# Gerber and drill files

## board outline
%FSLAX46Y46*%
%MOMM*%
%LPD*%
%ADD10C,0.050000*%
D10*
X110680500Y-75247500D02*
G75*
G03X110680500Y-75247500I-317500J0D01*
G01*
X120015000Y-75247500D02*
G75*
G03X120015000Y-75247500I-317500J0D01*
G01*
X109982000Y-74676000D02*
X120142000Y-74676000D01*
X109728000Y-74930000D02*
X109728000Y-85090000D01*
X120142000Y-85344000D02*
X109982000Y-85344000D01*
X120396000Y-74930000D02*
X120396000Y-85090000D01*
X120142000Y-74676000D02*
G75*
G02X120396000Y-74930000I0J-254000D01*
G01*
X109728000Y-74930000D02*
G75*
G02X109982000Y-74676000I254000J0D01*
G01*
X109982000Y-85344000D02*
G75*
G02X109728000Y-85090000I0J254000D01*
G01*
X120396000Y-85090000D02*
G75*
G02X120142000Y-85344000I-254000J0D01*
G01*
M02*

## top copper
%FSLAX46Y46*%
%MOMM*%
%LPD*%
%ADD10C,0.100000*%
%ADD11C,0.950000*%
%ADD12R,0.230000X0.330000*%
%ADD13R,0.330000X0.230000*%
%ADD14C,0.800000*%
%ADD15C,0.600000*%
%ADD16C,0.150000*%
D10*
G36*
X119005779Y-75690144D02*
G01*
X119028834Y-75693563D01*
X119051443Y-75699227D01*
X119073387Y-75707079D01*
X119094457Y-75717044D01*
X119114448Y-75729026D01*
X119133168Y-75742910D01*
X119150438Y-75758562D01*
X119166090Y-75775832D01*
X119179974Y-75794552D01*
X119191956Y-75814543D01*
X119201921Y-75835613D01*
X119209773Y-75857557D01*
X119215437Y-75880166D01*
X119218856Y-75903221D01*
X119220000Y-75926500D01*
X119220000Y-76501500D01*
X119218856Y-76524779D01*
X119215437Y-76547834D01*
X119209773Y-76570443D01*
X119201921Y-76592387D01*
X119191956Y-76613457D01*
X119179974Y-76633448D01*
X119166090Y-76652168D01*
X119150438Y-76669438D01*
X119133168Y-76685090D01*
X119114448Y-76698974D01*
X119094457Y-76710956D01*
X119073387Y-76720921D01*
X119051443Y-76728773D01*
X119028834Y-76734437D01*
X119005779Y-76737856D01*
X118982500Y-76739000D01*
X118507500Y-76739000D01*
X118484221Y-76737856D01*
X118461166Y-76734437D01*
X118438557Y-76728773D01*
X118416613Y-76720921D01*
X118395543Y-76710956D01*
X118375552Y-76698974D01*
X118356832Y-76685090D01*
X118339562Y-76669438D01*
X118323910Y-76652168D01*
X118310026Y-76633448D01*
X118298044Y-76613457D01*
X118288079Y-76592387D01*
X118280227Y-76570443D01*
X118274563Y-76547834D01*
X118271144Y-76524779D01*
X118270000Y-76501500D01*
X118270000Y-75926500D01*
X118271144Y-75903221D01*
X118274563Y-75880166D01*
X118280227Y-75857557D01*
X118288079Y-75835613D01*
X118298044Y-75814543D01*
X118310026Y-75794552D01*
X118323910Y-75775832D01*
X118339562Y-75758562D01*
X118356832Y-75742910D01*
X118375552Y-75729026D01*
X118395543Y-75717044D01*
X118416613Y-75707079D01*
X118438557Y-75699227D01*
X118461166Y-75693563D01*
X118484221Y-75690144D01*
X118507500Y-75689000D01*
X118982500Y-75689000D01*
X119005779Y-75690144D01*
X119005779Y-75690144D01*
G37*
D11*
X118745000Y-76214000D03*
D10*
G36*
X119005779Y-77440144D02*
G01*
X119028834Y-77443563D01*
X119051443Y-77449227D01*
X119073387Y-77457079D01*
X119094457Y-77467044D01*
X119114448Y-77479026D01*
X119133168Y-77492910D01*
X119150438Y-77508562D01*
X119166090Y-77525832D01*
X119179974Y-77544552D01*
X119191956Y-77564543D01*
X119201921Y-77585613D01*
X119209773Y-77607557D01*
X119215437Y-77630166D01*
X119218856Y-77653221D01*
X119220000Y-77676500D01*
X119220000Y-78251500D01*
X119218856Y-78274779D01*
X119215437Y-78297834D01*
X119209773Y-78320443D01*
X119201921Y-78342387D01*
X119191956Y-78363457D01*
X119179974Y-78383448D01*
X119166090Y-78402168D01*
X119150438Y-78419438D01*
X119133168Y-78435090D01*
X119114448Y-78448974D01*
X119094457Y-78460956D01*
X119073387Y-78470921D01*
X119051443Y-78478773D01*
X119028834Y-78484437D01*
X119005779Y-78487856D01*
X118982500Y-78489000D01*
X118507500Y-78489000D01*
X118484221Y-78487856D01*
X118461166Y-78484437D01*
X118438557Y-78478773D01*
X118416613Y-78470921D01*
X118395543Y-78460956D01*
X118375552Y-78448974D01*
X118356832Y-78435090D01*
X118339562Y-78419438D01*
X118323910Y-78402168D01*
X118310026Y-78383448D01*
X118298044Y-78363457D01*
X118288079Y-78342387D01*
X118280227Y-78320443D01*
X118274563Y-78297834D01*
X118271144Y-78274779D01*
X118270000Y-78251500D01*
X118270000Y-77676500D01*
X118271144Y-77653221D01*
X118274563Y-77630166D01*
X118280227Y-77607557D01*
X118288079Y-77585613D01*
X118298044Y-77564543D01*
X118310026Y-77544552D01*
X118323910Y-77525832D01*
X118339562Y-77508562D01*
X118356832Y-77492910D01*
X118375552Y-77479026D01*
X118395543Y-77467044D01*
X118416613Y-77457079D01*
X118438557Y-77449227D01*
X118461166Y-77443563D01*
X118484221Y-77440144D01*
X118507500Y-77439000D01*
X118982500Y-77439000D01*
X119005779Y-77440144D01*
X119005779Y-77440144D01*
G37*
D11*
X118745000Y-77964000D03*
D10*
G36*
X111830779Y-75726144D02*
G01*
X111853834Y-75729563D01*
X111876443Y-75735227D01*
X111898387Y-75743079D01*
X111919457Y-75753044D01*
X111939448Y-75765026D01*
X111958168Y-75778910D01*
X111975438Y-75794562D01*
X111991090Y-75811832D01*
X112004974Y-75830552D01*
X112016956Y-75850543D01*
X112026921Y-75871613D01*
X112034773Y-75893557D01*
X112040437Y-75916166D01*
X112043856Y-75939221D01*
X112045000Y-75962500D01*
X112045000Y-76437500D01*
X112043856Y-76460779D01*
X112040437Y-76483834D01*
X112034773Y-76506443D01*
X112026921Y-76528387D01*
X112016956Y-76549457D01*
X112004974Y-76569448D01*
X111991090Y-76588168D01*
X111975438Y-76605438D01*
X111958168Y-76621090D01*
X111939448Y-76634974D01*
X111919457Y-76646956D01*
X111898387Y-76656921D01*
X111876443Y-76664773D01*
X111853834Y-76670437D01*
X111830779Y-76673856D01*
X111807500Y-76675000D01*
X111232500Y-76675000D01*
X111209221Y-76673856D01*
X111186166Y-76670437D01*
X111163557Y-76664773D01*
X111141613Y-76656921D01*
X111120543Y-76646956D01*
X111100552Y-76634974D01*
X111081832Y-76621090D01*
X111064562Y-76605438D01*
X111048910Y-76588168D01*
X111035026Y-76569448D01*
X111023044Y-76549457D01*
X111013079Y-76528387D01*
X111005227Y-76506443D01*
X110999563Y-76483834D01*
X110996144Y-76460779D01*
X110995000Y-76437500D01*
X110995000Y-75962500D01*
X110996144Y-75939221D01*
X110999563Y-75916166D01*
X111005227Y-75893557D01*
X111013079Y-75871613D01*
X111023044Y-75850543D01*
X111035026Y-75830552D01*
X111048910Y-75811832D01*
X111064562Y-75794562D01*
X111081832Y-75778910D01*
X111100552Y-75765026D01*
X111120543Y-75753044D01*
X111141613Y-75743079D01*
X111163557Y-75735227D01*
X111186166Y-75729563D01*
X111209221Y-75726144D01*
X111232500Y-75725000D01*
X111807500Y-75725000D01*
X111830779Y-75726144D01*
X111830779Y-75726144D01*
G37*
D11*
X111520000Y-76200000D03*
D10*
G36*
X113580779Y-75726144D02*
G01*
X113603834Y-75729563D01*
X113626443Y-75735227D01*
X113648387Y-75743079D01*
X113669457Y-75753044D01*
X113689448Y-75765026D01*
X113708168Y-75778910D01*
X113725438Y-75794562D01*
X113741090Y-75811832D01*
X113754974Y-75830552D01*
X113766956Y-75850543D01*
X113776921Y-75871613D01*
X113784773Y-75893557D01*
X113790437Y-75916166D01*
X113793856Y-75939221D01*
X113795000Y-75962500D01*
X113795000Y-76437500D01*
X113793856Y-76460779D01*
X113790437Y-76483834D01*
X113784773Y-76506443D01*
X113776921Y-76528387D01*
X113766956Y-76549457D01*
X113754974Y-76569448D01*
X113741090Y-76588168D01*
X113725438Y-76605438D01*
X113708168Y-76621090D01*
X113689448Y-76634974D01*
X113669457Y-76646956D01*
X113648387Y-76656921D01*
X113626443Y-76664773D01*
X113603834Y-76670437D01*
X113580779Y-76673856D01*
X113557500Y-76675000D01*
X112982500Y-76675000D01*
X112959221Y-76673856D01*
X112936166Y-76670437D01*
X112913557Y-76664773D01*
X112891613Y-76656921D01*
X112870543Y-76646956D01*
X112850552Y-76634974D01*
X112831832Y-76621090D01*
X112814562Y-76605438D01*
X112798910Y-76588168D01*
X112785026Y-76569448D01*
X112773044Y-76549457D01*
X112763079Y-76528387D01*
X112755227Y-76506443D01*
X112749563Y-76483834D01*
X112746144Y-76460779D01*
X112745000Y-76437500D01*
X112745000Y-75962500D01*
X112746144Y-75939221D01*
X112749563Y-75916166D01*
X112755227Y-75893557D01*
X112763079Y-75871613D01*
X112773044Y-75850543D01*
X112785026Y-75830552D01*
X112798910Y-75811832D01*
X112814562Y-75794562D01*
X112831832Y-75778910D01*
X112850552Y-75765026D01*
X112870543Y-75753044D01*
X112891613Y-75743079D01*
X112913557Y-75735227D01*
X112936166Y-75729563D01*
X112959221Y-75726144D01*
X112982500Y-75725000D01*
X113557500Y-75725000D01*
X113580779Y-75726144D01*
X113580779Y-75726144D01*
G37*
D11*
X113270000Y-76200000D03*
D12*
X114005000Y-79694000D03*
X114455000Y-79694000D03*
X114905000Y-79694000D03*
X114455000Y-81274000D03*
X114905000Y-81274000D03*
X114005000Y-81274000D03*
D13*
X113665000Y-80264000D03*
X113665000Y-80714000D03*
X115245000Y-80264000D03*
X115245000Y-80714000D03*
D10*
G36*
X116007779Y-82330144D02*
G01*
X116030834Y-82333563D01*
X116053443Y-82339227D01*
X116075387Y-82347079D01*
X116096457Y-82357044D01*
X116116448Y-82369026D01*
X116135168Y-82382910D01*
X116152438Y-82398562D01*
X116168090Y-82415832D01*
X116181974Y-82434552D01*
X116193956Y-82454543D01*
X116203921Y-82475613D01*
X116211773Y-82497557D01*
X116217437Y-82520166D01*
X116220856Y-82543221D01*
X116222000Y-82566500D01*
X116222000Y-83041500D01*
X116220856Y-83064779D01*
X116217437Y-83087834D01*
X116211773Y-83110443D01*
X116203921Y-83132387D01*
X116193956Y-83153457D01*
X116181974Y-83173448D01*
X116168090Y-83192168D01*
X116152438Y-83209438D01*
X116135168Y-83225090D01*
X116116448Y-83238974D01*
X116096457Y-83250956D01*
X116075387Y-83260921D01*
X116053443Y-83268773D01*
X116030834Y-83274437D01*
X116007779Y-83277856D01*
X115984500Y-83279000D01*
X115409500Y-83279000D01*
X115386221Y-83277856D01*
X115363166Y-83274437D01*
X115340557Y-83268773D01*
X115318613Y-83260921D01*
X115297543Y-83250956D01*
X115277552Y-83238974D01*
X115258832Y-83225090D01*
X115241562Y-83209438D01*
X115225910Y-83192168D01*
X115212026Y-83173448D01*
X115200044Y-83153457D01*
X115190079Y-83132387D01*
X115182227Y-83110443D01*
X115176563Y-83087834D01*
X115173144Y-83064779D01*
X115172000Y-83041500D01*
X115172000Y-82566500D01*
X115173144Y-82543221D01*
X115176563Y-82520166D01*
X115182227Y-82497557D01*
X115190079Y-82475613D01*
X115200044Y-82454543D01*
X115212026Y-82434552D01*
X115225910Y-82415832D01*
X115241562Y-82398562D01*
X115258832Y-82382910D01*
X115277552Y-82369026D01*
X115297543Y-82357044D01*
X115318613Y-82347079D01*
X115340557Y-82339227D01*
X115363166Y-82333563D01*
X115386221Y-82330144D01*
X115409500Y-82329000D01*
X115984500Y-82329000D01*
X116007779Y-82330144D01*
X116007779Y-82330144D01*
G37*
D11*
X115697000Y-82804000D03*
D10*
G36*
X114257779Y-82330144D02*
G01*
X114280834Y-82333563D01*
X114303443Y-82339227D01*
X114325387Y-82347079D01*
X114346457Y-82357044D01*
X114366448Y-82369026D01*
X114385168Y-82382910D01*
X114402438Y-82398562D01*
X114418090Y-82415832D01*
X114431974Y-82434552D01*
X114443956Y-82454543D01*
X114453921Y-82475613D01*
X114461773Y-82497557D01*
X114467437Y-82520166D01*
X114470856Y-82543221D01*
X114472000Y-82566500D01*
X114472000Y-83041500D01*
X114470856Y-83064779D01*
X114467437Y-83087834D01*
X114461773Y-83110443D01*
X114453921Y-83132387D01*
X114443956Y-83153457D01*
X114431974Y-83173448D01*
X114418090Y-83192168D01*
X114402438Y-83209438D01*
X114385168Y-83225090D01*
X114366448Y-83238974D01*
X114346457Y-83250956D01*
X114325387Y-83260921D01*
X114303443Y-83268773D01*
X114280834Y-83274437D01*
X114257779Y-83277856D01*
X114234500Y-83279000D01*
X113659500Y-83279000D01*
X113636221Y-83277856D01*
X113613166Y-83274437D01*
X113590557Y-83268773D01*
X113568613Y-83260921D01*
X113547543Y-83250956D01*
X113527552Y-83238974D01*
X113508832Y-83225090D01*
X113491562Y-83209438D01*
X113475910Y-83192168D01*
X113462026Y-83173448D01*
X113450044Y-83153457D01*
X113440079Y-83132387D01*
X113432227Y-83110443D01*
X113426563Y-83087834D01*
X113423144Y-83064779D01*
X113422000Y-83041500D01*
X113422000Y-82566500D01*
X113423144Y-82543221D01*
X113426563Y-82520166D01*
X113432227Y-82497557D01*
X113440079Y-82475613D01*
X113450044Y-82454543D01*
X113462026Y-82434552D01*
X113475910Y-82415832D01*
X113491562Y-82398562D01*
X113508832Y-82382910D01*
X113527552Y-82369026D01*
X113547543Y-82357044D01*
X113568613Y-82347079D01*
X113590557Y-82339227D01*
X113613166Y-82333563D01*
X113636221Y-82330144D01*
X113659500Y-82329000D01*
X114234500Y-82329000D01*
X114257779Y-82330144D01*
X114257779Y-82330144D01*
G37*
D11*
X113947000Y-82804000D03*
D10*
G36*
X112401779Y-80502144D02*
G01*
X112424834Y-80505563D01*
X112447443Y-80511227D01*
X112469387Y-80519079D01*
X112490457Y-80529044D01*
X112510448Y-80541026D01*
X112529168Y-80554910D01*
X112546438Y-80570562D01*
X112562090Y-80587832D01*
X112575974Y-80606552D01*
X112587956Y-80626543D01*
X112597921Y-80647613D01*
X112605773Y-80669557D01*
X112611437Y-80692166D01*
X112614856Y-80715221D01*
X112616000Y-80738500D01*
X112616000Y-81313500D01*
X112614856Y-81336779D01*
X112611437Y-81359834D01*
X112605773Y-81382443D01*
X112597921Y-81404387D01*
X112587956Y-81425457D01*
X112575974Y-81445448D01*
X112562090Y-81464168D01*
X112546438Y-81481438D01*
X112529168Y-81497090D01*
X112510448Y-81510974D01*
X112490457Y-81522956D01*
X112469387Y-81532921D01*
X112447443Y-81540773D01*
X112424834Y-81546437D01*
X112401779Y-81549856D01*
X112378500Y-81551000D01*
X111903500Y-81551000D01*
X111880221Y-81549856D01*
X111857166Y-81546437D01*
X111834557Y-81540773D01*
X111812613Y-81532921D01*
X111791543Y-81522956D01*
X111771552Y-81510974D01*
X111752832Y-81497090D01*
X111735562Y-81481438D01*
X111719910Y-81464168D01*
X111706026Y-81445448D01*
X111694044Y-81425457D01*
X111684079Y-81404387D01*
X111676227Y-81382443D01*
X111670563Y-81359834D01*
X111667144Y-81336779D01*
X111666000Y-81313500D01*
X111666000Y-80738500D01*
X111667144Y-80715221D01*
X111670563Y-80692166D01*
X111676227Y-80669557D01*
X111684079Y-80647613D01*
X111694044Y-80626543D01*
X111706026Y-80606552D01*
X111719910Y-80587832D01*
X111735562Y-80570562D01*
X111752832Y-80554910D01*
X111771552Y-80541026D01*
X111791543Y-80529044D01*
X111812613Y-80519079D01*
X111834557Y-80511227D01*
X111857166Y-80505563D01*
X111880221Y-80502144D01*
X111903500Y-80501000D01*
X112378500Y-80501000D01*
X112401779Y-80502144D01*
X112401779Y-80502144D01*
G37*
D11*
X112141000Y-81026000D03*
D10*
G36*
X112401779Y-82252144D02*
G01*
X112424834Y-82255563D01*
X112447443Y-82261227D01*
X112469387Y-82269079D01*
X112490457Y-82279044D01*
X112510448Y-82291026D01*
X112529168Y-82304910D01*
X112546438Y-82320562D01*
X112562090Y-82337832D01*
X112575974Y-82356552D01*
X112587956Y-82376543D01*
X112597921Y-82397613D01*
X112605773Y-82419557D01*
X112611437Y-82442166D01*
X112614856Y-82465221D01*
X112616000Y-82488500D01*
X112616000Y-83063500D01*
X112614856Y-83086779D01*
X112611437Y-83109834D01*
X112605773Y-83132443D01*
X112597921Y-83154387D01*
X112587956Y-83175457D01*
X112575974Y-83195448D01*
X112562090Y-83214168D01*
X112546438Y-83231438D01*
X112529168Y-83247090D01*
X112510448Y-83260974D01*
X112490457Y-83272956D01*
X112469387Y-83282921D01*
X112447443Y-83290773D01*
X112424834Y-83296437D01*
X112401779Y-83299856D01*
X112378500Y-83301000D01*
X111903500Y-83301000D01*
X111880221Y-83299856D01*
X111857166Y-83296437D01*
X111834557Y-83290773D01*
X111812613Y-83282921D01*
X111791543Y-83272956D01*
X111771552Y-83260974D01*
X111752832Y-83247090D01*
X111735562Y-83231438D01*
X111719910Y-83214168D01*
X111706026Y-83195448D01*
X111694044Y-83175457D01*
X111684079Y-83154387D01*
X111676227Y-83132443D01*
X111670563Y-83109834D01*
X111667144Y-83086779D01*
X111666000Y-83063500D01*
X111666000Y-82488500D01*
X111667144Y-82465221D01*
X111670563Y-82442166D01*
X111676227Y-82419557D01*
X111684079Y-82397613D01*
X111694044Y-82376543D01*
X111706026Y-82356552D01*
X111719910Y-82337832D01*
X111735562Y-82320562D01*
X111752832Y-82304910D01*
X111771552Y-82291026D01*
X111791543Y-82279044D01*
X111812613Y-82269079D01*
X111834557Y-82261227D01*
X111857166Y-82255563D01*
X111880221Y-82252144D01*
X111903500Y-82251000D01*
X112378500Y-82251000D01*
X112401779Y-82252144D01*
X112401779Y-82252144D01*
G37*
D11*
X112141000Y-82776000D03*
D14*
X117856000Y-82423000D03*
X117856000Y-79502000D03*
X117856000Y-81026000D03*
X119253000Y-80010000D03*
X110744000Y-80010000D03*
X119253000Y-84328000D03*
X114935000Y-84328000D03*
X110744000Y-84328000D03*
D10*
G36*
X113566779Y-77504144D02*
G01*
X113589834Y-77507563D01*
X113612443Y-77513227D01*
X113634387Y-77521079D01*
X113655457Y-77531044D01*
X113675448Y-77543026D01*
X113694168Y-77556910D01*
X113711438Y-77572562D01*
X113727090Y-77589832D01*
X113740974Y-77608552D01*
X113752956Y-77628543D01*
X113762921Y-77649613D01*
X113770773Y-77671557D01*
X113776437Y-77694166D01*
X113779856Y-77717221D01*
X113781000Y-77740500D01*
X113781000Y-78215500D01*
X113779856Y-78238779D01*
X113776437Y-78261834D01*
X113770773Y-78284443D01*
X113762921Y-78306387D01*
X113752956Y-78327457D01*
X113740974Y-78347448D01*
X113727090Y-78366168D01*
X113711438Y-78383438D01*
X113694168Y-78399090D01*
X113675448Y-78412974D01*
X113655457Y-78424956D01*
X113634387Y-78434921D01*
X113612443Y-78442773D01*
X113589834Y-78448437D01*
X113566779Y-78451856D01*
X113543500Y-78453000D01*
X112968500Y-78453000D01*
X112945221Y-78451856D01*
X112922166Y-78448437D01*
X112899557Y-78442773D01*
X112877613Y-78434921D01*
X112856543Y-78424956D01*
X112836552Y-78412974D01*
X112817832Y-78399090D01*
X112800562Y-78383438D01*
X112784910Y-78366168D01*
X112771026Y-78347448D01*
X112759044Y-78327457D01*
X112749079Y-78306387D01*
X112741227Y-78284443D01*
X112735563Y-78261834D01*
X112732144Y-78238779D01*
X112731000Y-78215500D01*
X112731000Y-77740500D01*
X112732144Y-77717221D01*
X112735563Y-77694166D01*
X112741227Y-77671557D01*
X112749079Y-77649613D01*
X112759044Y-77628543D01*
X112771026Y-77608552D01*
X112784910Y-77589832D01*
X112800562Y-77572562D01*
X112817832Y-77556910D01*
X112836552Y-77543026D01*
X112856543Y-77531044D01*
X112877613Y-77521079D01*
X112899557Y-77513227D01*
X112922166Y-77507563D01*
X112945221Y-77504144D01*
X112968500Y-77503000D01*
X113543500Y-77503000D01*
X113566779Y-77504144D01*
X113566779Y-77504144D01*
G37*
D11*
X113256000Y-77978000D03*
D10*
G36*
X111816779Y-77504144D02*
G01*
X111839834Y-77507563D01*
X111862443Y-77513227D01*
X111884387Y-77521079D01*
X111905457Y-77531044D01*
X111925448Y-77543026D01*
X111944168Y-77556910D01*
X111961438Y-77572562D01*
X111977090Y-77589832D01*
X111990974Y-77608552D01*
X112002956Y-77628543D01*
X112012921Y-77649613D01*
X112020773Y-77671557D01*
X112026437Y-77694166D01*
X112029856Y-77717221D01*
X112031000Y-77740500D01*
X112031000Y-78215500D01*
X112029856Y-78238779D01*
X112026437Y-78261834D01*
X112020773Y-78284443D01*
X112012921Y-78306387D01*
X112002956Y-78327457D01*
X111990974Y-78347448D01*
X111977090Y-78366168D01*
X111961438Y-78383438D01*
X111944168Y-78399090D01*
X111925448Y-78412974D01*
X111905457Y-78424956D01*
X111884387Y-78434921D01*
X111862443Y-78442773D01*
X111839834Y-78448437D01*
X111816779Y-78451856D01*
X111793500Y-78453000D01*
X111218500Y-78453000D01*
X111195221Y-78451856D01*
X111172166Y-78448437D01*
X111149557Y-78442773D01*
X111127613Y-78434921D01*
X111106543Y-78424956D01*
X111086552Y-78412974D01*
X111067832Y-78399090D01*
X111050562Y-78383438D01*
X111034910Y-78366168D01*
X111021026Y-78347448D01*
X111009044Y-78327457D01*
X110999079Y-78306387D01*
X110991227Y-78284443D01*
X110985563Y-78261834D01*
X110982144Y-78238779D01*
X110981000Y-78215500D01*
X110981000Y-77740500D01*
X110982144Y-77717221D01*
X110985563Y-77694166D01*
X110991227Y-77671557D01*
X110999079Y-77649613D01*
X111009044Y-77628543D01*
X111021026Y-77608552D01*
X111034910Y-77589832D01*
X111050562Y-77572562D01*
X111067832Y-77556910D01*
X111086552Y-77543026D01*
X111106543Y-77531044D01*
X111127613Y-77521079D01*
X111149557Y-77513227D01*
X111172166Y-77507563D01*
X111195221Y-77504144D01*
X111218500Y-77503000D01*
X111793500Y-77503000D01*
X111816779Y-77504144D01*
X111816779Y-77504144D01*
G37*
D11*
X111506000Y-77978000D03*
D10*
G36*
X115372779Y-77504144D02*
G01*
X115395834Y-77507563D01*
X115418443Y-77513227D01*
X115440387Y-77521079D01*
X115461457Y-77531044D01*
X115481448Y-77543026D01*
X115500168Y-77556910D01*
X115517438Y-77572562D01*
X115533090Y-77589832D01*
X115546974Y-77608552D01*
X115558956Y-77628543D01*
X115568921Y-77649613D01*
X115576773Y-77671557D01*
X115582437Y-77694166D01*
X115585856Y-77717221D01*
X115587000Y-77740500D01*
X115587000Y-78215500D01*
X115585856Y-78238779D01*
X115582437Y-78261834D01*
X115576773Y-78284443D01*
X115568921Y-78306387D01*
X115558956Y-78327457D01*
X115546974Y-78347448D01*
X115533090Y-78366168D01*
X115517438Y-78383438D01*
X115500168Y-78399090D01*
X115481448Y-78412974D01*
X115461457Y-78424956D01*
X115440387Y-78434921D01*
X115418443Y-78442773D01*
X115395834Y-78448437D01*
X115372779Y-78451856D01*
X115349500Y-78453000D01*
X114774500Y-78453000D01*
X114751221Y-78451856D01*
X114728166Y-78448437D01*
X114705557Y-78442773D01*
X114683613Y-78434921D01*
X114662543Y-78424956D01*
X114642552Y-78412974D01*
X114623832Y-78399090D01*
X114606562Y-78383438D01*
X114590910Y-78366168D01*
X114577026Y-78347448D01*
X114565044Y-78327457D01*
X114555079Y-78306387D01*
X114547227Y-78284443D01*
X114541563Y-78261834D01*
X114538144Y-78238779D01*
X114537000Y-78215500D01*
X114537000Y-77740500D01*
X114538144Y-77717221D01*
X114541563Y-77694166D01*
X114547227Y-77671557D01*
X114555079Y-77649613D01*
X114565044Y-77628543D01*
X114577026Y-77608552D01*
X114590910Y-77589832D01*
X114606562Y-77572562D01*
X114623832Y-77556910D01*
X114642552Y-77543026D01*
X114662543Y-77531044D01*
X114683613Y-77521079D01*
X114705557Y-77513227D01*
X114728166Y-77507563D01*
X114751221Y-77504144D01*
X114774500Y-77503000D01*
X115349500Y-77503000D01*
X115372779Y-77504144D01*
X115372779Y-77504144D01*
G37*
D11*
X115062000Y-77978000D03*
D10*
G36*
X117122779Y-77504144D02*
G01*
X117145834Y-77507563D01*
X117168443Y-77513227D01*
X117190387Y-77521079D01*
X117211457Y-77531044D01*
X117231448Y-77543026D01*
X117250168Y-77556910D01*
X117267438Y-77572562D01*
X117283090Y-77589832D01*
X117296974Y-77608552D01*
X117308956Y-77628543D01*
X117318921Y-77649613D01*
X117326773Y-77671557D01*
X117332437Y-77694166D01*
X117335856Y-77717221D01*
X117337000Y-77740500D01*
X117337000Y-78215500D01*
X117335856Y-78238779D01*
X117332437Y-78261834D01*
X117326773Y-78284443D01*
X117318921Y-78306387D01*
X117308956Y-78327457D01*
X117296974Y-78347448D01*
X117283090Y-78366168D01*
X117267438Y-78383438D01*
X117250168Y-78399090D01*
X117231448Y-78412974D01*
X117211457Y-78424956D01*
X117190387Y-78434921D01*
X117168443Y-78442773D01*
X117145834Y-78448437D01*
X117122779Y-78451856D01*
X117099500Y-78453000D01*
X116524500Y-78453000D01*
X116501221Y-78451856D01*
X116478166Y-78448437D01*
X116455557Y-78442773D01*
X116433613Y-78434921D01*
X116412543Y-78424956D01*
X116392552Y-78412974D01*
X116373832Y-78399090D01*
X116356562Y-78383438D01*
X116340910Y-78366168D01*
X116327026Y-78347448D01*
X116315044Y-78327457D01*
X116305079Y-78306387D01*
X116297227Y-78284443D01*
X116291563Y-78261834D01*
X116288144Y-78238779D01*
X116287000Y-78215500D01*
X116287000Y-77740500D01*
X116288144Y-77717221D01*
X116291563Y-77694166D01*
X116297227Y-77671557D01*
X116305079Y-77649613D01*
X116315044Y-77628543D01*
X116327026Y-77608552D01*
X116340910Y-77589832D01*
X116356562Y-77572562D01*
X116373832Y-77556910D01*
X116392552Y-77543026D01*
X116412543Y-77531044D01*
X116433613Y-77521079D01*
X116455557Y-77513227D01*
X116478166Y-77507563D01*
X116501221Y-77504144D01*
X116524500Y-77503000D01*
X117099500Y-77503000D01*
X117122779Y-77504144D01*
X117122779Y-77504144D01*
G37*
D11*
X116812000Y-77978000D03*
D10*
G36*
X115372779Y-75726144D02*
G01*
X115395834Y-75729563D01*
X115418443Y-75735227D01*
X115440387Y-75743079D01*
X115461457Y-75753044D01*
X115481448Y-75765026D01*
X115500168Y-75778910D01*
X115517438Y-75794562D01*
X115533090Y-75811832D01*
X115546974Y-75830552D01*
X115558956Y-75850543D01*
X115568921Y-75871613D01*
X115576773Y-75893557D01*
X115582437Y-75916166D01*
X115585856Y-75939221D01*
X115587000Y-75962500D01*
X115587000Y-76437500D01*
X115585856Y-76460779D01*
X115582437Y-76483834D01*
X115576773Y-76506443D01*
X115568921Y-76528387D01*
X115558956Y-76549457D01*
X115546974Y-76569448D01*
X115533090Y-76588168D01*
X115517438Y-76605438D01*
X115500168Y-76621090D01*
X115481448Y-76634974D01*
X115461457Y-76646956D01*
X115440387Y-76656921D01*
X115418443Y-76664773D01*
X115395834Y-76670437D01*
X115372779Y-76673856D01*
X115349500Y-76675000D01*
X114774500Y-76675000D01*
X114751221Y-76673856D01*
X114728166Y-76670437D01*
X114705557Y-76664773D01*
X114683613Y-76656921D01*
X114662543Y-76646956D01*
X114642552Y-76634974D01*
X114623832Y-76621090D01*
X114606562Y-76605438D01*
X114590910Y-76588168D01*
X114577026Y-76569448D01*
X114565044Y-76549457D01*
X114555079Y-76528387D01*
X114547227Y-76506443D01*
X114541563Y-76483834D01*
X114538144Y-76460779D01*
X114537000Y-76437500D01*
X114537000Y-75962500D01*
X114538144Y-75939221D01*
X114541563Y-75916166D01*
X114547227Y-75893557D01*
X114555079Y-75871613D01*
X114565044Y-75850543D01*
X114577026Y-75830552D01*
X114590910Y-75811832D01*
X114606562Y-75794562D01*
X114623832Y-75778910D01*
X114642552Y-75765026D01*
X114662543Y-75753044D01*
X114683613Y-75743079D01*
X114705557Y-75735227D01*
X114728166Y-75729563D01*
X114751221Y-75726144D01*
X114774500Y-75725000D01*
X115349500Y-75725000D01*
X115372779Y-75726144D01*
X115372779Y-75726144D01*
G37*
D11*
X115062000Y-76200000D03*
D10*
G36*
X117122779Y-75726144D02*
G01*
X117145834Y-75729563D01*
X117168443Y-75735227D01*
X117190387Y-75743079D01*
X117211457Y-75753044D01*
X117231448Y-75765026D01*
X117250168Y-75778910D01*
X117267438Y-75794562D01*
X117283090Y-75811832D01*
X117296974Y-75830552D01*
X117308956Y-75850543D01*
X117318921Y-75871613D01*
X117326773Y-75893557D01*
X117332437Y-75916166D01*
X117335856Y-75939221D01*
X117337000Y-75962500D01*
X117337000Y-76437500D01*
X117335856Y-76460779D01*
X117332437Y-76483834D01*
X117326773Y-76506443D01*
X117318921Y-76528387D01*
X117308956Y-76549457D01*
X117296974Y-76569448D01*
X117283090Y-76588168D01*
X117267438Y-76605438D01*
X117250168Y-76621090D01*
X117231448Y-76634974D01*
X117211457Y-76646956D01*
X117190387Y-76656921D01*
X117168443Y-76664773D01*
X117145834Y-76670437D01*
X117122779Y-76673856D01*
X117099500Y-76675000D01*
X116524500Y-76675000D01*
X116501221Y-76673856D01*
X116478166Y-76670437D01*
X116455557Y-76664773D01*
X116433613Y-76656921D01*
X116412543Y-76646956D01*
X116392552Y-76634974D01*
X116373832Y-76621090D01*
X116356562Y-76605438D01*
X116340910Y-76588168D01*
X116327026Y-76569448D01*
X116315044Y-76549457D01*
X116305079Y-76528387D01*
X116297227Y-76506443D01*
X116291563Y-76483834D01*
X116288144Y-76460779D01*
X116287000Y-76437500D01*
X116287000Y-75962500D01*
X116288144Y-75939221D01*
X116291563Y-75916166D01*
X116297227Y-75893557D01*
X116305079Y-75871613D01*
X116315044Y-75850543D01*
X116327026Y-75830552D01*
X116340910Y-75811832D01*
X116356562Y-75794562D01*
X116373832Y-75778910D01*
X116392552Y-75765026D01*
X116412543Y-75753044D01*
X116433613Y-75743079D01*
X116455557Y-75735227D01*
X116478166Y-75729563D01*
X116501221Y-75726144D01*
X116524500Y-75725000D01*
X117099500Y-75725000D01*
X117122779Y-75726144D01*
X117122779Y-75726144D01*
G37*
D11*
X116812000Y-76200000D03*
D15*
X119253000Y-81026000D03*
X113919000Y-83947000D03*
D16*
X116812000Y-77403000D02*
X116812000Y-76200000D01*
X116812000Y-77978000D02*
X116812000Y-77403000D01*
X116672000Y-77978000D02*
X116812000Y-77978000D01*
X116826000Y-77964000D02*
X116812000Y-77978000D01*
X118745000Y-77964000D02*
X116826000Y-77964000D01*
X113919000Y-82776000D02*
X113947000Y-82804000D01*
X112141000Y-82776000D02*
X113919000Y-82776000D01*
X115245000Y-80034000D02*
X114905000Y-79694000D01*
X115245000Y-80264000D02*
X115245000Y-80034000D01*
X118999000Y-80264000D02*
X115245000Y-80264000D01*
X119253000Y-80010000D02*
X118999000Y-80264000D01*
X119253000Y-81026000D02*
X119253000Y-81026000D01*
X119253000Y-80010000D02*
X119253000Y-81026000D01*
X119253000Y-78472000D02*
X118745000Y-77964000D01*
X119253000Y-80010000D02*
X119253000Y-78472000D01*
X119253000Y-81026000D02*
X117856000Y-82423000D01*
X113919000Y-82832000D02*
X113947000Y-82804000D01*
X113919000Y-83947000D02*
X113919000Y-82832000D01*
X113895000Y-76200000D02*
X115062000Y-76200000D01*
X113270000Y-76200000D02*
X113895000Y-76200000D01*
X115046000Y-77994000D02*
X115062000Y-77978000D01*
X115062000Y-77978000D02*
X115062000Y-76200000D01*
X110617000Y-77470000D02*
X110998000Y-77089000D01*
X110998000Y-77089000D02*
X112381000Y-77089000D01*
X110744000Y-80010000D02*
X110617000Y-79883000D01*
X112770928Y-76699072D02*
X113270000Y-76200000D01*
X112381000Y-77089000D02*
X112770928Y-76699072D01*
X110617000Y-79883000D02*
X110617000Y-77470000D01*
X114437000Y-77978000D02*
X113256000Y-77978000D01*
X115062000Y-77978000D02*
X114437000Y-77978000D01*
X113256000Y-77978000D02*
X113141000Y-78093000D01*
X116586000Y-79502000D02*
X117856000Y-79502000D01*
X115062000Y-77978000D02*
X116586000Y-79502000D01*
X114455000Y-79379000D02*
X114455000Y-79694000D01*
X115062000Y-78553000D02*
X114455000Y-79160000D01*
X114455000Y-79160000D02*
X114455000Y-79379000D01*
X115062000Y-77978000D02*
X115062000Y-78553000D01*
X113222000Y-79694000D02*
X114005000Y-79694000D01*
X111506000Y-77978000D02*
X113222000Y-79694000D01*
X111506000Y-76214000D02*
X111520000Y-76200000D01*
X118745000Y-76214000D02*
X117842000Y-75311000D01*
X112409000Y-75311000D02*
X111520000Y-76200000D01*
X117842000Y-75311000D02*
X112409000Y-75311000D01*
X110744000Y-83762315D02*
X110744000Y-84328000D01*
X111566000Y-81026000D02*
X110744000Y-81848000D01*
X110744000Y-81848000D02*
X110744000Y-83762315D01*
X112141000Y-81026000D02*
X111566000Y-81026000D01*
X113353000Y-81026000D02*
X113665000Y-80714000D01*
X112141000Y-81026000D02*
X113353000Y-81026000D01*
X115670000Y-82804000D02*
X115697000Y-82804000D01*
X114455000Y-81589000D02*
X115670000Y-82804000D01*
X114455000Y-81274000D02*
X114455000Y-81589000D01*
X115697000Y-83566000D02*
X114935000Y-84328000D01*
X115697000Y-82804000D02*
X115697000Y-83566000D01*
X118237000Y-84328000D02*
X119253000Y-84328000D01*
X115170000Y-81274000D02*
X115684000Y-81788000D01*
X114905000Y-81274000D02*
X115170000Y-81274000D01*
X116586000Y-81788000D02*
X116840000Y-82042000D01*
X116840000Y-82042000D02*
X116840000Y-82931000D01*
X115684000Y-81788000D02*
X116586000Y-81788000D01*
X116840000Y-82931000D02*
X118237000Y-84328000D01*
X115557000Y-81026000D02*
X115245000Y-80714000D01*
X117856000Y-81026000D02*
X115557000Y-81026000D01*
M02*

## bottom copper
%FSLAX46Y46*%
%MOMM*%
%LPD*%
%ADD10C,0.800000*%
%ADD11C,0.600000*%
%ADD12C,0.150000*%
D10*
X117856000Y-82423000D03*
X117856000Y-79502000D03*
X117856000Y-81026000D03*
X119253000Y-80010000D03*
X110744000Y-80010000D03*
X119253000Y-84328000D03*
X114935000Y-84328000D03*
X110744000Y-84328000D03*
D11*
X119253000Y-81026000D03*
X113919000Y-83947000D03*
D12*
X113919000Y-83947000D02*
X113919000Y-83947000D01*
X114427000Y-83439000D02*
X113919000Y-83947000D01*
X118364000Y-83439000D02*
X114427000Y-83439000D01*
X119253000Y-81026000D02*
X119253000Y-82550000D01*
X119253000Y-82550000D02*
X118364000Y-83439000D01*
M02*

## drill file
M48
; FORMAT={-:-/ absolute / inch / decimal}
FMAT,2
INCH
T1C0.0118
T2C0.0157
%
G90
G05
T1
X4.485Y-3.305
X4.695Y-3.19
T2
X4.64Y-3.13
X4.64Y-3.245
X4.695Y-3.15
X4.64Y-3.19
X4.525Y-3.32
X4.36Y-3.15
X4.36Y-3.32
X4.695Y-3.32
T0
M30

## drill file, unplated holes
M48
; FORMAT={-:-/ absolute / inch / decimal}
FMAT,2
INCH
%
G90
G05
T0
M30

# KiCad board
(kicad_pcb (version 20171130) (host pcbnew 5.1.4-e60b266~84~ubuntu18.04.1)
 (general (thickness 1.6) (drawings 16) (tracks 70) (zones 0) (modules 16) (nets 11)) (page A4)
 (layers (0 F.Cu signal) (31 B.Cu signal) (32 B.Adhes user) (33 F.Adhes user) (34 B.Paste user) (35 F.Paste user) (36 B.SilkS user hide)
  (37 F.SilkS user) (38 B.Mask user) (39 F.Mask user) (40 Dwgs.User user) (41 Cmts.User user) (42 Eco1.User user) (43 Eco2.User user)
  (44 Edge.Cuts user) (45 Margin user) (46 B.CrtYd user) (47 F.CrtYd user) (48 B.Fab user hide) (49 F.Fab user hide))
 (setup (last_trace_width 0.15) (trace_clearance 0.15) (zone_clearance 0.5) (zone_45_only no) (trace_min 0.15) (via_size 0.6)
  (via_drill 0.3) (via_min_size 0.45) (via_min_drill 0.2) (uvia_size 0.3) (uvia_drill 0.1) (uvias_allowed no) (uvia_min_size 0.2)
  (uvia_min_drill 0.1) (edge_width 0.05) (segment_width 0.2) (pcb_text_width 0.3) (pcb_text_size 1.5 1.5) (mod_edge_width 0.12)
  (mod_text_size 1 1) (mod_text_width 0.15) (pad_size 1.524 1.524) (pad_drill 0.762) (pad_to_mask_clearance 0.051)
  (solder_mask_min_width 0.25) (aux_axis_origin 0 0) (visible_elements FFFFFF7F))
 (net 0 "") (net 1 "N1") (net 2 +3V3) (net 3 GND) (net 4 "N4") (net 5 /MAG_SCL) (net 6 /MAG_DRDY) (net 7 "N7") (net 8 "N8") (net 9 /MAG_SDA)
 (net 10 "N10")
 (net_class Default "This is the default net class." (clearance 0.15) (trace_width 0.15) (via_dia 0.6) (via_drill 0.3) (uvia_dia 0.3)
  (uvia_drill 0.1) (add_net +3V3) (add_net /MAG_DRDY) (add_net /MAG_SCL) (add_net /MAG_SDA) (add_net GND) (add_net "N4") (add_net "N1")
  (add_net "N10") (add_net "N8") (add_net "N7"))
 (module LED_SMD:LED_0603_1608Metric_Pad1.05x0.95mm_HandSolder (layer F.Cu) (at 118.745 77.089 270)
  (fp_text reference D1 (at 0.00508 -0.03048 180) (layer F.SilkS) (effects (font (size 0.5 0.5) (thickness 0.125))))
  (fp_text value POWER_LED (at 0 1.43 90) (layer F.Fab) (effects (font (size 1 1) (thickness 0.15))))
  (pad 1 smd roundrect (at -0.875 0 270) (size 1.05 0.95) (layers F.Cu F.Paste F.Mask) (roundrect_rratio 0.25) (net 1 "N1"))
  (pad 2 smd roundrect (at 0.875 0 270) (size 1.05 0.95) (layers F.Cu F.Paste F.Mask) (roundrect_rratio 0.25) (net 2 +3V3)))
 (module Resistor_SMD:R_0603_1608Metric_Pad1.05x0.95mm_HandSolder (layer F.Cu) (at 112.395 76.2)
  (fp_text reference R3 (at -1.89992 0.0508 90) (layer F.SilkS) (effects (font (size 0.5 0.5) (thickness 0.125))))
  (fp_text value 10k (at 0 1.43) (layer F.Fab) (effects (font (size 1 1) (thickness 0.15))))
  (pad 1 smd roundrect (at -0.875 0) (size 1.05 0.95) (layers F.Cu F.Paste F.Mask) (roundrect_rratio 0.25) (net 1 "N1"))
  (pad 2 smd roundrect (at 0.875 0) (size 1.05 0.95) (layers F.Cu F.Paste F.Mask) (roundrect_rratio 0.25) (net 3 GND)))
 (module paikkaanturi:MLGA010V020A (layer F.Cu) (at 113.455 79.484)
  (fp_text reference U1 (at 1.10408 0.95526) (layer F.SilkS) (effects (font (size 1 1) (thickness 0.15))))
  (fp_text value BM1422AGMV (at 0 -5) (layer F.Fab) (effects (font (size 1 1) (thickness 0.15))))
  (pad 3 smd rect (at 0.55 0.21) (size 0.23 0.33) (layers F.Cu F.Paste F.Mask) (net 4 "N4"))
  (pad 2 smd rect (at 1 0.21) (size 0.23 0.33) (layers F.Cu F.Paste F.Mask) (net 3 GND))
  (pad 1 smd rect (at 1.45 0.21) (size 0.23 0.33) (layers F.Cu F.Paste F.Mask) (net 2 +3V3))
  (pad 7 smd rect (at 1 1.79) (size 0.23 0.33) (layers F.Cu F.Paste F.Mask) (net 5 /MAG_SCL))
  (pad 8 smd rect (at 1.45 1.79) (size 0.23 0.33) (layers F.Cu F.Paste F.Mask) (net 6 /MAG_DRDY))
  (pad 6 smd rect (at 0.55 1.79) (size 0.23 0.33) (layers F.Cu F.Paste F.Mask) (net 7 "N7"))
  (pad 4 smd rect (at 0.21 0.78 90) (size 0.23 0.33) (layers F.Cu F.Paste F.Mask) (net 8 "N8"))
  (pad 5 smd rect (at 0.21 1.23 90) (size 0.23 0.33) (layers F.Cu F.Paste F.Mask) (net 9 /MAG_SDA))
  (pad 10 smd rect (at 1.79 0.78 90) (size 0.23 0.33) (layers F.Cu F.Paste F.Mask) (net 2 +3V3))
  (pad 9 smd rect (at 1.79 1.23 90) (size 0.23 0.33) (layers F.Cu F.Paste F.Mask) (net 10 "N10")))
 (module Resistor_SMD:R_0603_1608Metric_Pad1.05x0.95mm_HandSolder (layer F.Cu) (at 114.822 82.804 180)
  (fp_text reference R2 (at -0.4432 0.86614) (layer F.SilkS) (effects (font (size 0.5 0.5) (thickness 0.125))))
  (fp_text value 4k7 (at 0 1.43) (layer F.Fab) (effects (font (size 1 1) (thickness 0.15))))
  (pad 1 smd roundrect (at -0.875 0 180) (size 1.05 0.95) (layers F.Cu F.Paste F.Mask) (roundrect_rratio 0.25) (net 5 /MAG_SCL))
  (pad 2 smd roundrect (at 0.875 0 180) (size 1.05 0.95) (layers F.Cu F.Paste F.Mask) (roundrect_rratio 0.25) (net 2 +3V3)))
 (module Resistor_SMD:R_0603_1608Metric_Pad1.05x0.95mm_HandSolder (layer F.Cu) (at 112.141 81.901 270)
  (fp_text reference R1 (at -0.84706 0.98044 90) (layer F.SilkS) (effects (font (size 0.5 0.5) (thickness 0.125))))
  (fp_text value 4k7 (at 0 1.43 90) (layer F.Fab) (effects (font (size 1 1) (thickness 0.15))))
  (pad 1 smd roundrect (at -0.875 0 270) (size 1.05 0.95) (layers F.Cu F.Paste F.Mask) (roundrect_rratio 0.25) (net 9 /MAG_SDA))
  (pad 2 smd roundrect (at 0.875 0 270) (size 1.05 0.95) (layers F.Cu F.Paste F.Mask) (roundrect_rratio 0.25) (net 2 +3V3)))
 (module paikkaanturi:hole (layer F.Cu) (at 117.856 82.423)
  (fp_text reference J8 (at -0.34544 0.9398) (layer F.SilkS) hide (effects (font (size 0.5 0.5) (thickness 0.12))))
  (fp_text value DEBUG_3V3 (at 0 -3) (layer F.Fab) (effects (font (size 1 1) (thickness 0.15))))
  (pad 1 thru_hole circle (at 0 0) (size 0.8 0.8) (drill 0.4) (layers *.Cu *.Mask) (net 2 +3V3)))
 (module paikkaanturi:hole (layer F.Cu) (at 117.856 79.502)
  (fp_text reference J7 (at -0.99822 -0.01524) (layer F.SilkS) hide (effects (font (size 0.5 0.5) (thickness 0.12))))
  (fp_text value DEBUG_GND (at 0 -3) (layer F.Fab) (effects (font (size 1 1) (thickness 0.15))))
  (pad 1 thru_hole circle (at 0 0) (size 0.8 0.8) (drill 0.4) (layers *.Cu *.Mask) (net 3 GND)))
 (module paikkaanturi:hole (layer F.Cu) (at 117.856 81.026)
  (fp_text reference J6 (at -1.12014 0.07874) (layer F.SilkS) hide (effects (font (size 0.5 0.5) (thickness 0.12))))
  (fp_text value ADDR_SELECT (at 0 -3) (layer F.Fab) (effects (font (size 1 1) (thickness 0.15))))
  (pad 1 thru_hole circle (at 0 0) (size 0.8 0.8) (drill 0.4) (layers *.Cu *.Mask) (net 10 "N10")))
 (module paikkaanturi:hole (layer F.Cu) (at 119.253 80.01)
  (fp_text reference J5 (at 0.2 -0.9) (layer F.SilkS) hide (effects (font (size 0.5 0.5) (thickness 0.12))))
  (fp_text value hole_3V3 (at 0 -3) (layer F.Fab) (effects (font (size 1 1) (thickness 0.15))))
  (pad 1 thru_hole circle (at 0 0) (size 0.8 0.8) (drill 0.4) (layers *.Cu *.Mask) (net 2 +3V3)))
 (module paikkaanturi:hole (layer F.Cu) (at 110.744 80.01)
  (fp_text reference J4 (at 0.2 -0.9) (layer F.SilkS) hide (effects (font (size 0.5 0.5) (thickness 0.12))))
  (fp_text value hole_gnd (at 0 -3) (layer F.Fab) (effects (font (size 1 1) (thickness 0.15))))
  (pad 1 thru_hole circle (at 0 0) (size 0.8 0.8) (drill 0.4) (layers *.Cu *.Mask) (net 3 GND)))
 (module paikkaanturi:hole (layer F.Cu) (at 119.253 84.328)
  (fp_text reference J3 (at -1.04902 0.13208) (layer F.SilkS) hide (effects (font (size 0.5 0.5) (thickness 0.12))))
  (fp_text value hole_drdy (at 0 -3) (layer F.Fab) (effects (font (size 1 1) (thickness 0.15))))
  (pad 1 thru_hole circle (at 0 0) (size 0.8 0.8) (drill 0.4) (layers *.Cu *.Mask) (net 6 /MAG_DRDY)))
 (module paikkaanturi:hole (layer F.Cu) (at 114.935 84.328)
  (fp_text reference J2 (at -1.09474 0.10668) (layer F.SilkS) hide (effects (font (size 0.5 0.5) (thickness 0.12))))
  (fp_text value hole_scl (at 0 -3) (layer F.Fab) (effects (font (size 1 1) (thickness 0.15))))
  (pad 1 thru_hole circle (at 0 0) (size 0.8 0.8) (drill 0.4) (layers *.Cu *.Mask) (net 5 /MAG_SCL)))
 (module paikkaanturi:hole (layer F.Cu) (at 110.744 84.328)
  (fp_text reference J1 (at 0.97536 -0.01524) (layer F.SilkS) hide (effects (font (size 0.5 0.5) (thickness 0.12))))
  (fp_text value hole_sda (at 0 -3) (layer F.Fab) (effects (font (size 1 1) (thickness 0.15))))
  (pad 1 thru_hole circle (at 0 0) (size 0.8 0.8) (drill 0.4) (layers *.Cu *.Mask) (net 9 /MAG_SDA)))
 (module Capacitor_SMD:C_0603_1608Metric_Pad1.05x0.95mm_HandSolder (layer F.Cu) (at 112.381 77.978 180)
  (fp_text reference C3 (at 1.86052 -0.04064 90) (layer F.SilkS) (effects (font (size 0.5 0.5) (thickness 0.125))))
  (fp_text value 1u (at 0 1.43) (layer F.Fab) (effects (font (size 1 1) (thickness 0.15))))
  (pad 1 smd roundrect (at -0.875 0 180) (size 1.05 0.95) (layers F.Cu F.Paste F.Mask) (roundrect_rratio 0.25) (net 3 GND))
  (pad 2 smd roundrect (at 0.875 0 180) (size 1.05 0.95) (layers F.Cu F.Paste F.Mask) (roundrect_rratio 0.25) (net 4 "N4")))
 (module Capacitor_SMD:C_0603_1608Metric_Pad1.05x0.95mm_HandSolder (layer F.Cu) (at 115.937 77.978)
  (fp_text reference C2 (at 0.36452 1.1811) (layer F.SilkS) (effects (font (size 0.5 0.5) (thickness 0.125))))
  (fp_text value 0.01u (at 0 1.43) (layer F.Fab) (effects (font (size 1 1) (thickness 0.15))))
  (pad 1 smd roundrect (at -0.875 0) (size 1.05 0.95) (layers F.Cu F.Paste F.Mask) (roundrect_rratio 0.25) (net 3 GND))
  (pad 2 smd roundrect (at 0.875 0) (size 1.05 0.95) (layers F.Cu F.Paste F.Mask) (roundrect_rratio 0.25) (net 2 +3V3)))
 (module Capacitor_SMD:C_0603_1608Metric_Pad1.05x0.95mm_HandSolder (layer F.Cu) (at 115.937 76.2)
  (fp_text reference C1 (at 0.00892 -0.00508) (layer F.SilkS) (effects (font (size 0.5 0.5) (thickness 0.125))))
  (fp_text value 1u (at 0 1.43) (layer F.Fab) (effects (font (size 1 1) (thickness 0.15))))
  (pad 1 smd roundrect (at -0.875 0) (size 1.05 0.95) (layers F.Cu F.Paste F.Mask) (roundrect_rratio 0.25) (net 3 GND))
  (pad 2 smd roundrect (at 0.875 0) (size 1.05 0.95) (layers F.Cu F.Paste F.Mask) (roundrect_rratio 0.25) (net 2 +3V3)))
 (gr_circle (center 110.363 75.2475) (end 110.617 75.057) (layer Edge.Cuts) (width 0.05))
 (gr_circle (center 119.6975 75.2475) (end 119.9515 75.057) (layer Edge.Cuts) (width 0.05))
 (gr_line (start 109.982 74.676) (end 120.142 74.676) (layer Edge.Cuts) (width 0.05))
 (gr_line (start 109.728 74.93) (end 109.728 85.09) (layer Edge.Cuts) (width 0.05))
 (gr_line (start 120.142 85.344) (end 109.982 85.344) (layer Edge.Cuts) (width 0.05))
 (gr_line (start 120.396 74.93) (end 120.396 85.09) (layer Edge.Cuts) (width 0.05))
 (gr_arc (start 120.142 74.93) (end 120.396 74.93) (angle -90) (layer Edge.Cuts) (width 0.05))
 (gr_arc (start 109.982 74.93) (end 109.982 74.676) (angle -90) (layer Edge.Cuts) (width 0.05))
 (gr_arc (start 109.982 85.09) (end 109.728 85.09) (angle -90) (layer Edge.Cuts) (width 0.05))
 (gr_arc (start 120.142 85.09) (end 120.142 85.344) (angle -90) (layer Edge.Cuts) (width 0.05))
 (segment (start 116.812 77.403) (end 116.812 76.2) (width 0.15) (layer F.Cu) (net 2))
 (segment (start 116.812 77.978) (end 116.812 77.403) (width 0.15) (layer F.Cu) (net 2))
 (segment (start 116.672 77.978) (end 116.812 77.978) (width 0.15) (layer F.Cu) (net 2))
 (segment (start 116.826 77.964) (end 116.812 77.978) (width 0.15) (layer F.Cu) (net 2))
 (segment (start 118.745 77.964) (end 116.826 77.964) (width 0.15) (layer F.Cu) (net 2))
 (segment (start 113.919 82.776) (end 113.947 82.804) (width 0.15) (layer F.Cu) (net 2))
 (segment (start 112.141 82.776) (end 113.919 82.776) (width 0.15) (layer F.Cu) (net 2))
 (segment (start 115.245 80.034) (end 114.905 79.694) (width 0.15) (layer F.Cu) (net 2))
 (segment (start 115.245 80.264) (end 115.245 80.034) (width 0.15) (layer F.Cu) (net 2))
 (segment (start 118.999 80.264) (end 115.245 80.264) (width 0.15) (layer F.Cu) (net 2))
 (segment (start 119.253 80.01) (end 118.999 80.264) (width 0.15) (layer F.Cu) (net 2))
 (segment (start 119.253 81.026) (end 119.253 81.026) (width 0.15) (layer F.Cu) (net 2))
 (segment (start 119.253 80.01) (end 119.253 81.026) (width 0.15) (layer F.Cu) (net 2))
 (segment (start 119.253 78.472) (end 118.745 77.964) (width 0.15) (layer F.Cu) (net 2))
 (segment (start 119.253 80.01) (end 119.253 78.472) (width 0.15) (layer F.Cu) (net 2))
 (segment (start 119.253 81.026) (end 117.856 82.423) (width 0.15) (layer F.Cu) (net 2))
 (via (at 119.253 81.026) (size 0.6) (drill 0.3) (layers F.Cu B.Cu) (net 2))
 (segment (start 113.919 83.947) (end 113.919 83.947) (width 0.15) (layer B.Cu) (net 2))
 (via (at 113.919 83.947) (size 0.6) (drill 0.3) (layers F.Cu B.Cu) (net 2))
 (segment (start 113.919 82.832) (end 113.947 82.804) (width 0.15) (layer F.Cu) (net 2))
 (segment (start 113.919 83.947) (end 113.919 82.832) (width 0.15) (layer F.Cu) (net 2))
 (segment (start 114.427 83.439) (end 113.919 83.947) (width 0.15) (layer B.Cu) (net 2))
 (segment (start 118.364 83.439) (end 114.427 83.439) (width 0.15) (layer B.Cu) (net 2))
 (segment (start 119.253 81.026) (end 119.253 82.55) (width 0.15) (layer B.Cu) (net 2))
 (segment (start 119.253 82.55) (end 118.364 83.439) (width 0.15) (layer B.Cu) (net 2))
 (segment (start 113.895 76.2) (end 115.062 76.2) (width 0.15) (layer F.Cu) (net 3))
 (segment (start 113.27 76.2) (end 113.895 76.2) (width 0.15) (layer F.Cu) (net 3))
 (segment (start 115.046 77.994) (end 115.062 77.978) (width 0.15) (layer F.Cu) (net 3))
 (segment (start 115.062 77.978) (end 115.062 76.2) (width 0.15) (layer F.Cu) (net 3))
 (segment (start 110.617 77.47) (end 110.998 77.089) (width 0.15) (layer F.Cu) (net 3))
 (segment (start 110.998 77.089) (end 112.381 77.089) (width 0.15) (layer F.Cu) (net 3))
 (segment (start 110.744 80.01) (end 110.617 79.883) (width 0.15) (layer F.Cu) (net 3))
 (segment (start 112.770928 76.699072) (end 113.27 76.2) (width 0.15) (layer F.Cu) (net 3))
 (segment (start 112.381 77.089) (end 112.770928 76.699072) (width 0.15) (layer F.Cu) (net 3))
 (segment (start 110.617 79.883) (end 110.617 77.47) (width 0.15) (layer F.Cu) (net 3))
 (segment (start 114.437 77.978) (end 113.256 77.978) (width 0.15) (layer F.Cu) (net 3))
 (segment (start 115.062 77.978) (end 114.437 77.978) (width 0.15) (layer F.Cu) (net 3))
 (segment (start 113.256 77.978) (end 113.141 78.093) (width 0.15) (layer F.Cu) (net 3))
 (segment (start 116.586 79.502) (end 117.856 79.502) (width 0.15) (layer F.Cu) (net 3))
 (segment (start 115.062 77.978) (end 116.586 79.502) (width 0.15) (layer F.Cu) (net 3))
 (segment (start 114.455 79.379) (end 114.455 79.694) (width 0.15) (layer F.Cu) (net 3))
 (segment (start 115.062 78.553) (end 114.455 79.16) (width 0.15) (layer F.Cu) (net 3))
 (segment (start 114.455 79.16) (end 114.455 79.379) (width 0.15) (layer F.Cu) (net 3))
 (segment (start 115.062 77.978) (end 115.062 78.553) (width 0.15) (layer F.Cu) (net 3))
 (segment (start 113.222 79.694) (end 114.005 79.694) (width 0.15) (layer F.Cu) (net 4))
 (segment (start 111.506 77.978) (end 113.222 79.694) (width 0.15) (layer F.Cu) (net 4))
 (segment (start 111.506 76.214) (end 111.52 76.2) (width 0.15) (layer F.Cu) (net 1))
 (segment (start 118.745 76.214) (end 117.842 75.311) (width 0.15) (layer F.Cu) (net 1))
 (segment (start 112.409 75.311) (end 111.52 76.2) (width 0.15) (layer F.Cu) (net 1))
 (segment (start 117.842 75.311) (end 112.409 75.311) (width 0.15) (layer F.Cu) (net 1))
 (segment (start 110.744 83.762315) (end 110.744 84.328) (width 0.15) (layer F.Cu) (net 9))
 (segment (start 111.566 81.026) (end 110.744 81.848) (width 0.15) (layer F.Cu) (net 9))
 (segment (start 110.744 81.848) (end 110.744 83.762315) (width 0.15) (layer F.Cu) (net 9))
 (segment (start 112.141 81.026) (end 111.566 81.026) (width 0.15) (layer F.Cu) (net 9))
 (segment (start 113.353 81.026) (end 113.665 80.714) (width 0.15) (layer F.Cu) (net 9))
 (segment (start 112.141 81.026) (end 113.353 81.026) (width 0.15) (layer F.Cu) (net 9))
 (segment (start 115.67 82.804) (end 115.697 82.804) (width 0.15) (layer F.Cu) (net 5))
 (segment (start 114.455 81.589) (end 115.67 82.804) (width 0.15) (layer F.Cu) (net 5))
 (segment (start 114.455 81.274) (end 114.455 81.589) (width 0.15) (layer F.Cu) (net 5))
 (segment (start 115.697 83.566) (end 114.935 84.328) (width 0.15) (layer F.Cu) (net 5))
 (segment (start 115.697 82.804) (end 115.697 83.566) (width 0.15) (layer F.Cu) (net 5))
 (segment (start 118.237 84.328) (end 119.253 84.328) (width 0.15) (layer F.Cu) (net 6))
 (segment (start 115.17 81.274) (end 115.684 81.788) (width 0.15) (layer F.Cu) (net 6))
 (segment (start 114.905 81.274) (end 115.17 81.274) (width 0.15) (layer F.Cu) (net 6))
 (segment (start 116.586 81.788) (end 116.84 82.042) (width 0.15) (layer F.Cu) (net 6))
 (segment (start 116.84 82.042) (end 116.84 82.931) (width 0.15) (layer F.Cu) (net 6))
 (segment (start 115.684 81.788) (end 116.586 81.788) (width 0.15) (layer F.Cu) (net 6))
 (segment (start 116.84 82.931) (end 118.237 84.328) (width 0.15) (layer F.Cu) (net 6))
 (segment (start 115.557 81.026) (end 115.245 80.714) (width 0.15) (layer F.Cu) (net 10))
 (segment (start 117.856 81.026) (end 115.557 81.026) (width 0.15) (layer F.Cu) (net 10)))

